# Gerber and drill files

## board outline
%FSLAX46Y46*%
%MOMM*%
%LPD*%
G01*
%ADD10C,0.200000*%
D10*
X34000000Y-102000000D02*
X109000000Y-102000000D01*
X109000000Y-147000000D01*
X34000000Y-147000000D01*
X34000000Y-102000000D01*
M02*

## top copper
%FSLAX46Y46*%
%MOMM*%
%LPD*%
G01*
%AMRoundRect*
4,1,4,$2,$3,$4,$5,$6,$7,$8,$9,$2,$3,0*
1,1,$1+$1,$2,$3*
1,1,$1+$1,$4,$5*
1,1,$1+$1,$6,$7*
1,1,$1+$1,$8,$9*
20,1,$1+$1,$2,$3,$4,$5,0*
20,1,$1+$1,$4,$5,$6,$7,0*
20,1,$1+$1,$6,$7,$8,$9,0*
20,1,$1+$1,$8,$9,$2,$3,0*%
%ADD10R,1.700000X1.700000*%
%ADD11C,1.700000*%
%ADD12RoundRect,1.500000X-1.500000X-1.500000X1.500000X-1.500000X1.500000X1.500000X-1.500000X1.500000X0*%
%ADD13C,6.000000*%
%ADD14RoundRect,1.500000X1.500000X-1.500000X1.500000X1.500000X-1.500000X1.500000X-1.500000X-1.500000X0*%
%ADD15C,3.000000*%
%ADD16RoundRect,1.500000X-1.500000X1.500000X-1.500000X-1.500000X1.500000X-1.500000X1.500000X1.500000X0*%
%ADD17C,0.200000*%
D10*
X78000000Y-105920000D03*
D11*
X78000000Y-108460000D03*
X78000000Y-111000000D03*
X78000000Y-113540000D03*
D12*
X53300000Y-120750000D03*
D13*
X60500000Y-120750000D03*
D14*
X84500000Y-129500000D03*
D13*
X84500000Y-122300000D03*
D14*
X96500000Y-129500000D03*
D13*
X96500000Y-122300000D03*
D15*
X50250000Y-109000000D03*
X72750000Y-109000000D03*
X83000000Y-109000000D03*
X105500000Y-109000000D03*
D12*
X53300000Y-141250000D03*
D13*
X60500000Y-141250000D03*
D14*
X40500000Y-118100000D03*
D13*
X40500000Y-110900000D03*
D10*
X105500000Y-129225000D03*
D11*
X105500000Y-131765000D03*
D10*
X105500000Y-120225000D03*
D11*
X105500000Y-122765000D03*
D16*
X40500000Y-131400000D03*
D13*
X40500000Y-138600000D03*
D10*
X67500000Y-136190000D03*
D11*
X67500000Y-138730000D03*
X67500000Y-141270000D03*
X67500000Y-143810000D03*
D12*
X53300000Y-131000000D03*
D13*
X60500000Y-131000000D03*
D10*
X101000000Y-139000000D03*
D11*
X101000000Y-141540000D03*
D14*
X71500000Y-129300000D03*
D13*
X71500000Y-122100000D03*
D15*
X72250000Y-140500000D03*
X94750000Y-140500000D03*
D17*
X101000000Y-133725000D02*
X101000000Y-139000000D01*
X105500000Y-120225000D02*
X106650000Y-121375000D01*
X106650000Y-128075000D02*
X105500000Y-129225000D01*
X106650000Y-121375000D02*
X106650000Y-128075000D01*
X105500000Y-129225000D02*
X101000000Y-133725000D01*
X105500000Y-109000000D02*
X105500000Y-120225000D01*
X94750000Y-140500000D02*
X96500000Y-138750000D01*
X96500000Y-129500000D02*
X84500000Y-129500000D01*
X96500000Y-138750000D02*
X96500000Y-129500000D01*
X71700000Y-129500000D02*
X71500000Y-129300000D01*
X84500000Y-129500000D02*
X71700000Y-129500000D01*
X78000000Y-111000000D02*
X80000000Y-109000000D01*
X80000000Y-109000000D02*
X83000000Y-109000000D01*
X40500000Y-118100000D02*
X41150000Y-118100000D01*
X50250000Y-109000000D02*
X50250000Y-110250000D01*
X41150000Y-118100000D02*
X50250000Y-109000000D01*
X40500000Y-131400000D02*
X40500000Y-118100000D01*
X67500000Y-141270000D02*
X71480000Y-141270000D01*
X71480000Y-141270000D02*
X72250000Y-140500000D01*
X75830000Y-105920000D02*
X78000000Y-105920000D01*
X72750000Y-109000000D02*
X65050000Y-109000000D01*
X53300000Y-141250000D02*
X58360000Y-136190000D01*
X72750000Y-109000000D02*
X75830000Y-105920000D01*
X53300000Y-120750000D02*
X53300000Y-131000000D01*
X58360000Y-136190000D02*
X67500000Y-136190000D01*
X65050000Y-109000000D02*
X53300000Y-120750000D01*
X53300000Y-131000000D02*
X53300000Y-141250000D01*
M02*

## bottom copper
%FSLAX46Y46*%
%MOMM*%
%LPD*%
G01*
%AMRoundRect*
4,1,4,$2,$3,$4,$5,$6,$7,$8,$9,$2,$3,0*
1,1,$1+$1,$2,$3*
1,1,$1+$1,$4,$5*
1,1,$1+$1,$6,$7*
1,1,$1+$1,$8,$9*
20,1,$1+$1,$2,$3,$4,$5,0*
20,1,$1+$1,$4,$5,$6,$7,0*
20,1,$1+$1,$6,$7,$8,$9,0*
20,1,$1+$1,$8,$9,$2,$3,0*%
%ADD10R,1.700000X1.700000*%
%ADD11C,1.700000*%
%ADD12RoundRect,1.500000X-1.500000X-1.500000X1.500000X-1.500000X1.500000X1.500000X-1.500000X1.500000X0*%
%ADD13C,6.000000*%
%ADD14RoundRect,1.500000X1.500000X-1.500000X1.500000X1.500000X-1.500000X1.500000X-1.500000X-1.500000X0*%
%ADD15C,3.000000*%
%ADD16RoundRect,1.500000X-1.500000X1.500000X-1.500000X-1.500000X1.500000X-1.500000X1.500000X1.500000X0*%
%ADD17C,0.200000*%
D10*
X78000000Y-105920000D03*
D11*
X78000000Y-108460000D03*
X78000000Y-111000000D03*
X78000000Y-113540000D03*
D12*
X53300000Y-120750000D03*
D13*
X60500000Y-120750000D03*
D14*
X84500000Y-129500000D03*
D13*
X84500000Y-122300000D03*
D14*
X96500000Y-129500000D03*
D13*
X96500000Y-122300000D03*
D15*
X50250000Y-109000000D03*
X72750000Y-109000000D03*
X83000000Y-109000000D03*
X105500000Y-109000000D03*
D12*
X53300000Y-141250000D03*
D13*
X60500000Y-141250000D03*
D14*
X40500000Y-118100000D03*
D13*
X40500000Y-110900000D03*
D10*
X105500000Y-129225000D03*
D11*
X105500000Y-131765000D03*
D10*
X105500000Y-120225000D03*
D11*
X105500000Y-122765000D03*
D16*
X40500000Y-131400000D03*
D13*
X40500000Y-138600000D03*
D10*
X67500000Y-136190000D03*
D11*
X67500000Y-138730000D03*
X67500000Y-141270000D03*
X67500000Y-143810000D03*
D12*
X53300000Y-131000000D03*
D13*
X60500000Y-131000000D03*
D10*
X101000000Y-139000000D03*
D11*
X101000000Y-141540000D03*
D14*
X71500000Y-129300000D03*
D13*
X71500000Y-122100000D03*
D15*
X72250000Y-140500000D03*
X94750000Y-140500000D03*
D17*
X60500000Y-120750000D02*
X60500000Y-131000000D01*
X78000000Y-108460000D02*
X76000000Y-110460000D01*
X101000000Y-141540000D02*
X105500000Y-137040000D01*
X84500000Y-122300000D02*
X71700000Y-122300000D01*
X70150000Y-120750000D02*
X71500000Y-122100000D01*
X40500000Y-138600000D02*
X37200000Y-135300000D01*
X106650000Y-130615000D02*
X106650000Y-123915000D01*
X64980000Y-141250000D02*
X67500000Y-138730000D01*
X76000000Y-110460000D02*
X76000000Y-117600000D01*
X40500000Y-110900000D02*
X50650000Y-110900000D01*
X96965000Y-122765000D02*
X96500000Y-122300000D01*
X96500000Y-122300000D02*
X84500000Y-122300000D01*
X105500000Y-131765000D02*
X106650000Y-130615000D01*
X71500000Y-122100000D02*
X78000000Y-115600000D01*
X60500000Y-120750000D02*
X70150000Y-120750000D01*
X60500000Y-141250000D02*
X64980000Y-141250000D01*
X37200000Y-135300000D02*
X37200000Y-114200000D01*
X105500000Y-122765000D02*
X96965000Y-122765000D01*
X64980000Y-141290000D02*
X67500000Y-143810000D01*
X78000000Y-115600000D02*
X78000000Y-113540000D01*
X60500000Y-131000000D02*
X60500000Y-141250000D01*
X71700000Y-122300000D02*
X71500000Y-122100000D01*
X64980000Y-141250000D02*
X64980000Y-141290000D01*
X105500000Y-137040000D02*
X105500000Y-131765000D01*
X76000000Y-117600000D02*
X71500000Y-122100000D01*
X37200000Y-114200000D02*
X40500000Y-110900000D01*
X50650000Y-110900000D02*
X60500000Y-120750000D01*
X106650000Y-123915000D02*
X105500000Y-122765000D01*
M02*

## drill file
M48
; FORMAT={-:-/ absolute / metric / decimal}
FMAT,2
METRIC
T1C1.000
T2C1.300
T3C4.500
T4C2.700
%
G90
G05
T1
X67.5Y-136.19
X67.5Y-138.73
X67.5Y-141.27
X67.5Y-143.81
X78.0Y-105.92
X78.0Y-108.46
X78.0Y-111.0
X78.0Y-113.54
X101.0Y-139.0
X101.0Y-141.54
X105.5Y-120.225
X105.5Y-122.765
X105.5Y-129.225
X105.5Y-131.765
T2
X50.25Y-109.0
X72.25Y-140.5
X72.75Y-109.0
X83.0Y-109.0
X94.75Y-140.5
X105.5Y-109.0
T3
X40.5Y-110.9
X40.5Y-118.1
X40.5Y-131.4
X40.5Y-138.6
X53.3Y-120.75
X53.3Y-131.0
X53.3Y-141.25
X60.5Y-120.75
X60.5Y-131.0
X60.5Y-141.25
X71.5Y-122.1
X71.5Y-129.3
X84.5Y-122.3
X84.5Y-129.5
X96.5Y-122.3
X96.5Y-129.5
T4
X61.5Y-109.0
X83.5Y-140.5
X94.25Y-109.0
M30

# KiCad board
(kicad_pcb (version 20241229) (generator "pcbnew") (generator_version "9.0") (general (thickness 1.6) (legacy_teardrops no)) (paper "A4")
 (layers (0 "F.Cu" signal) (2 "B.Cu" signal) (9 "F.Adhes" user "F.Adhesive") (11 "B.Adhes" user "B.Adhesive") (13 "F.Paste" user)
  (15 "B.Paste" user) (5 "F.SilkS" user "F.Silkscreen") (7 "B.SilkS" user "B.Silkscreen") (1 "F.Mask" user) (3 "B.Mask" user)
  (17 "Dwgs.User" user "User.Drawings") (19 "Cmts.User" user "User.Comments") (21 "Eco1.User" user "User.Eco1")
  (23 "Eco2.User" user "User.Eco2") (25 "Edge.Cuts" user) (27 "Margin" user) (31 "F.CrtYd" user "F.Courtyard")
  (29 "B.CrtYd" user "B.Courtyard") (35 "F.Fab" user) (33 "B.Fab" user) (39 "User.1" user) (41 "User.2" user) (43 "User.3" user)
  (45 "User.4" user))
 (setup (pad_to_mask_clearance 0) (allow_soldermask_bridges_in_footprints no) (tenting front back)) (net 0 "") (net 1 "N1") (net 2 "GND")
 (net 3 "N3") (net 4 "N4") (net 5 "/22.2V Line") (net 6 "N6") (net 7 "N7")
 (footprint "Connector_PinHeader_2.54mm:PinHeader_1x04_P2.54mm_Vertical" (layer "F.Cu") (at 78 105.92)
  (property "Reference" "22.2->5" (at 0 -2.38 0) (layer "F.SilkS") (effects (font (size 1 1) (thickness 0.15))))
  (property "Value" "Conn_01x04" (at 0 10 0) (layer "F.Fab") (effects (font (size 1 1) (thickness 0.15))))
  (pad "1" thru_hole rect (at 0 0) (size 1.7 1.7) (drill 1) (layers "*.Cu" "*.Mask") (remove_unused_layers no) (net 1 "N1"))
  (pad "2" thru_hole circle (at 0 2.54) (size 1.7 1.7) (drill 1) (layers "*.Cu" "*.Mask") (remove_unused_layers no) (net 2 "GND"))
  (pad "3" thru_hole circle (at 0 5.08) (size 1.7 1.7) (drill 1) (layers "*.Cu" "*.Mask") (remove_unused_layers no) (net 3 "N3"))
  (pad "4" thru_hole circle (at 0 7.62) (size 1.7 1.7) (drill 1) (layers "*.Cu" "*.Mask") (remove_unused_layers no) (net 2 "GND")))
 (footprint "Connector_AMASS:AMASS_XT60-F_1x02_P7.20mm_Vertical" (layer "F.Cu") (at 53.3 120.75)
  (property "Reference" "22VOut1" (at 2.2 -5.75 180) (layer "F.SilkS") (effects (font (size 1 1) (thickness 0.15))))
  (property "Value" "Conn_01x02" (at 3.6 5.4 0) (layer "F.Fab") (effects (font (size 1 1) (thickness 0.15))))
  (pad "1" thru_hole roundrect (at 0 0) (size 6 6) (drill 4.5) (layers "*.Cu" "*.Mask") (remove_unused_layers no) (roundrect_rratio 0.25)
   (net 1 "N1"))
  (pad "2" thru_hole circle (at 7.2 0) (size 6 6) (drill 4.5) (layers "*.Cu" "*.Mask") (remove_unused_layers no) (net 2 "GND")))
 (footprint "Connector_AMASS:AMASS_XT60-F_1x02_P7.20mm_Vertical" (layer "F.Cu") (at 84.5 129.5 90)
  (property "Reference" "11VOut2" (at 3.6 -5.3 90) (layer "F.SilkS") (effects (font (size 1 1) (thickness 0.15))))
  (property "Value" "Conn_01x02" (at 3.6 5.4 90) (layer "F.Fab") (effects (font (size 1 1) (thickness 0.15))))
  (pad "1" thru_hole roundrect (at 0 0 90) (size 6 6) (drill 4.5) (layers "*.Cu" "*.Mask") (remove_unused_layers no) (roundrect_rratio 0.25)
   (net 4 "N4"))
  (pad "2" thru_hole circle (at 7.2 0 90) (size 6 6) (drill 4.5) (layers "*.Cu" "*.Mask") (remove_unused_layers no) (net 2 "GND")))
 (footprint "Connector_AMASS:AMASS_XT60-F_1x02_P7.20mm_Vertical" (layer "F.Cu") (at 96.5 129.5 90)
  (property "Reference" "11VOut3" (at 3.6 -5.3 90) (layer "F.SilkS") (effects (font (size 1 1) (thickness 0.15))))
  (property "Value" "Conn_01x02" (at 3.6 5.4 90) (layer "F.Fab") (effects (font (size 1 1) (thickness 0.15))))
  (pad "1" thru_hole roundrect (at 0 0 90) (size 6 6) (drill 4.5) (layers "*.Cu" "*.Mask") (remove_unused_layers no) (roundrect_rratio 0.25)
   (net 4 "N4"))
  (pad "2" thru_hole circle (at 7.2 0 90) (size 6 6) (drill 4.5) (layers "*.Cu" "*.Mask") (remove_unused_layers no) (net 2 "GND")))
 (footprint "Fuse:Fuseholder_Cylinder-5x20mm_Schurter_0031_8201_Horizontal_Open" (layer "F.Cu") (at 50.25 109)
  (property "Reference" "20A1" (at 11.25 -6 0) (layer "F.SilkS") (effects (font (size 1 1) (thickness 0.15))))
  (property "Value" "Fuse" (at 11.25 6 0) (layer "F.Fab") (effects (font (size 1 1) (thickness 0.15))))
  (pad "" np_thru_hole circle (at 11.25 0) (size 2.7 2.7) (drill 2.7) (layers "*.Cu" "*.Mask"))
  (pad "1" thru_hole circle (at 0 0) (size 3 3) (drill 1.3) (layers "*.Cu" "*.Mask") (remove_unused_layers no) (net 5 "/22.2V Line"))
  (pad "2" thru_hole circle (at 22.5 0) (size 3 3) (drill 1.3) (layers "*.Cu" "*.Mask") (remove_unused_layers no) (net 1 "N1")))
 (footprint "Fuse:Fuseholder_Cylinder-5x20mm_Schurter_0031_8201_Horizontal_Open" (layer "F.Cu") (at 83 109)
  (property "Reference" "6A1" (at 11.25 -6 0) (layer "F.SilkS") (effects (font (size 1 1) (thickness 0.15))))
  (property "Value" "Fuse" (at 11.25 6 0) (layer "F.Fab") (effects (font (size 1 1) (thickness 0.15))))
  (pad "" np_thru_hole circle (at 11.25 0) (size 2.7 2.7) (drill 2.7) (layers "*.Cu" "*.Mask"))
  (pad "1" thru_hole circle (at 0 0) (size 3 3) (drill 1.3) (layers "*.Cu" "*.Mask") (remove_unused_layers no) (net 3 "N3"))
  (pad "2" thru_hole circle (at 22.5 0) (size 3 3) (drill 1.3) (layers "*.Cu" "*.Mask") (remove_unused_layers no) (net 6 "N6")))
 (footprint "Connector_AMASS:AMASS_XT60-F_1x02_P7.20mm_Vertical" (layer "F.Cu") (at 53.3 141.25)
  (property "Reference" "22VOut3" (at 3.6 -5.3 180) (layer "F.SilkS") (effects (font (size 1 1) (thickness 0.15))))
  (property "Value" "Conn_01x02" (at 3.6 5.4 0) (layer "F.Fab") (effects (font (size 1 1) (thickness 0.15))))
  (pad "1" thru_hole roundrect (at 0 0) (size 6 6) (drill 4.5) (layers "*.Cu" "*.Mask") (remove_unused_layers no) (roundrect_rratio 0.25)
   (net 1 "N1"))
  (pad "2" thru_hole circle (at 7.2 0) (size 6 6) (drill 4.5) (layers "*.Cu" "*.Mask") (remove_unused_layers no) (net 2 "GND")))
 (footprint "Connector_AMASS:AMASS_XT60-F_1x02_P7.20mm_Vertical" (layer "F.Cu") (at 40.5 118.1 90)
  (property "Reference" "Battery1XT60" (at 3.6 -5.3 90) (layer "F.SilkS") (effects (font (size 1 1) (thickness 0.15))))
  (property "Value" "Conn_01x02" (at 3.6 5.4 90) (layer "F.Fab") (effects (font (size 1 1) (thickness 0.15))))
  (pad "1" thru_hole roundrect (at 0 0 90) (size 6 6) (drill 4.5) (layers "*.Cu" "*.Mask") (remove_unused_layers no) (roundrect_rratio 0.25)
   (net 5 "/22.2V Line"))
  (pad "2" thru_hole circle (at 7.2 0 90) (size 6 6) (drill 4.5) (layers "*.Cu" "*.Mask") (remove_unused_layers no) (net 2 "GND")))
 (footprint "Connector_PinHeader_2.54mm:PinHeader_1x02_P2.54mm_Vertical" (layer "F.Cu") (at 105.5 129.225)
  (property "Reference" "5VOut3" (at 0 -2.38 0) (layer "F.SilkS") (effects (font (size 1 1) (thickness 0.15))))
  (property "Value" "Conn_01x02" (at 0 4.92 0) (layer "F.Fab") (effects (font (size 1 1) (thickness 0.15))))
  (pad "1" thru_hole rect (at 0 0) (size 1.7 1.7) (drill 1) (layers "*.Cu" "*.Mask") (remove_unused_layers no) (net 6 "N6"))
  (pad "2" thru_hole circle (at 0 2.54) (size 1.7 1.7) (drill 1) (layers "*.Cu" "*.Mask") (remove_unused_layers no) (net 2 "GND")))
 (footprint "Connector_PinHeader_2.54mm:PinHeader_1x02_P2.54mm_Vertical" (layer "F.Cu") (at 105.5 120.225)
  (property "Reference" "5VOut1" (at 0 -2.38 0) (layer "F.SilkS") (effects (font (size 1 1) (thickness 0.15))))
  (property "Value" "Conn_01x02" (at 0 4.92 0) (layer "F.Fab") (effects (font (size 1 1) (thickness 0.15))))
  (pad "1" thru_hole rect (at 0 0) (size 1.7 1.7) (drill 1) (layers "*.Cu" "*.Mask") (remove_unused_layers no) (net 6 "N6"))
  (pad "2" thru_hole circle (at 0 2.54) (size 1.7 1.7) (drill 1) (layers "*.Cu" "*.Mask") (remove_unused_layers no) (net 2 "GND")))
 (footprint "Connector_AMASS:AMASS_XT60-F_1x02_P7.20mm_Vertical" (layer "F.Cu") (at 40.5 131.4 -90)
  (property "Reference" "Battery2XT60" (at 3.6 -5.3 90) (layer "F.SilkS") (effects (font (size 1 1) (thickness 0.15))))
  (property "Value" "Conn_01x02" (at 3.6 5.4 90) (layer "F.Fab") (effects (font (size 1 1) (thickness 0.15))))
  (pad "1" thru_hole roundrect (at 0 0 270) (size 6 6) (drill 4.5) (layers "*.Cu" "*.Mask") (remove_unused_layers no)
   (roundrect_rratio 0.25) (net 5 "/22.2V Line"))
  (pad "2" thru_hole circle (at 7.2 0 270) (size 6 6) (drill 4.5) (layers "*.Cu" "*.Mask") (remove_unused_layers no) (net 2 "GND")))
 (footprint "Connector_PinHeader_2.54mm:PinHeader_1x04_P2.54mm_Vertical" (layer "F.Cu") (at 67.5 136.19)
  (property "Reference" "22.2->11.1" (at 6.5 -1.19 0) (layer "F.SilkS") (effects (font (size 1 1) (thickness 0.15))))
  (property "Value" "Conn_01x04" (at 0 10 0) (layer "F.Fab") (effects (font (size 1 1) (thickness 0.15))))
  (pad "1" thru_hole rect (at 0 0) (size 1.7 1.7) (drill 1) (layers "*.Cu" "*.Mask") (remove_unused_layers no) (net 1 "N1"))
  (pad "2" thru_hole circle (at 0 2.54) (size 1.7 1.7) (drill 1) (layers "*.Cu" "*.Mask") (remove_unused_layers no) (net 2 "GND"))
  (pad "3" thru_hole circle (at 0 5.08) (size 1.7 1.7) (drill 1) (layers "*.Cu" "*.Mask") (remove_unused_layers no) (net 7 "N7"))
  (pad "4" thru_hole circle (at 0 7.62) (size 1.7 1.7) (drill 1) (layers "*.Cu" "*.Mask") (remove_unused_layers no) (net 2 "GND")))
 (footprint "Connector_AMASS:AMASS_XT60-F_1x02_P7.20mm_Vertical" (layer "F.Cu") (at 53.3 131)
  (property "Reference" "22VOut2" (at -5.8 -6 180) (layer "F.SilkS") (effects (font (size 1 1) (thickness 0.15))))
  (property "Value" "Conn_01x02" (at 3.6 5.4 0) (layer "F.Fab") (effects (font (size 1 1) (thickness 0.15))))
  (pad "1" thru_hole roundrect (at 0 0) (size 6 6) (drill 4.5) (layers "*.Cu" "*.Mask") (remove_unused_layers no) (roundrect_rratio 0.25)
   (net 1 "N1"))
  (pad "2" thru_hole circle (at 7.2 0) (size 6 6) (drill 4.5) (layers "*.Cu" "*.Mask") (remove_unused_layers no) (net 2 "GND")))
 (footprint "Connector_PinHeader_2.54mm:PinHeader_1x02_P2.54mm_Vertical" (layer "F.Cu") (at 101 139)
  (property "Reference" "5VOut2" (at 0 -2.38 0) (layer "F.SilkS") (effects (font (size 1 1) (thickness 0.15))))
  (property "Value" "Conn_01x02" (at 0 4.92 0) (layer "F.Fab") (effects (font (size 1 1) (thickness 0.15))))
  (pad "1" thru_hole rect (at 0 0) (size 1.7 1.7) (drill 1) (layers "*.Cu" "*.Mask") (remove_unused_layers no) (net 6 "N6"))
  (pad "2" thru_hole circle (at 0 2.54) (size 1.7 1.7) (drill 1) (layers "*.Cu" "*.Mask") (remove_unused_layers no) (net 2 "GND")))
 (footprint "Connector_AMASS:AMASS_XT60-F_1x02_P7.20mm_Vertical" (layer "F.Cu") (at 71.5 129.3 90)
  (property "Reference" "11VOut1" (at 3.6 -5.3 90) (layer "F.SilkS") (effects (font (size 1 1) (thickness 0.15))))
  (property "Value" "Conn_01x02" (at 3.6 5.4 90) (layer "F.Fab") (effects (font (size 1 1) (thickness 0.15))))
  (pad "1" thru_hole roundrect (at 0 0 90) (size 6 6) (drill 4.5) (layers "*.Cu" "*.Mask") (remove_unused_layers no) (roundrect_rratio 0.25)
   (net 4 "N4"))
  (pad "2" thru_hole circle (at 7.2 0 90) (size 6 6) (drill 4.5) (layers "*.Cu" "*.Mask") (remove_unused_layers no) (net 2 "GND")))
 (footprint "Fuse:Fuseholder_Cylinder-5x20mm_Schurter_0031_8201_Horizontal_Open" (layer "F.Cu") (at 72.25 140.5)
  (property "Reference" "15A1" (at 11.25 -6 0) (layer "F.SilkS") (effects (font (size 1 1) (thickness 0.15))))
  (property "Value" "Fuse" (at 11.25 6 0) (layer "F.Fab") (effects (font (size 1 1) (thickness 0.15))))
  (pad "" np_thru_hole circle (at 11.25 0) (size 2.7 2.7) (drill 2.7) (layers "*.Cu" "*.Mask"))
  (pad "1" thru_hole circle (at 0 0) (size 3 3) (drill 1.3) (layers "*.Cu" "*.Mask") (remove_unused_layers no) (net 7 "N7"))
  (pad "2" thru_hole circle (at 22.5 0) (size 3 3) (drill 1.3) (layers "*.Cu" "*.Mask") (remove_unused_layers no) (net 4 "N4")))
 (gr_rect (start 34 102) (end 109 147) (stroke (width 0.2) (type solid)) (fill no) (layer "Edge.Cuts"))
 (segment (start 60.5 120.75) (end 60.5 131) (width 0.2) (layer "B.Cu") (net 2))
 (segment (start 78 108.46) (end 76 110.46) (width 0.2) (layer "B.Cu") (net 2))
 (segment (start 101 141.54) (end 105.5 137.04) (width 0.2) (layer "B.Cu") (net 2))
 (segment (start 84.5 122.3) (end 71.7 122.3) (width 0.2) (layer "B.Cu") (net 2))
 (segment (start 70.15 120.75) (end 71.5 122.1) (width 0.2) (layer "B.Cu") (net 2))
 (segment (start 40.5 138.6) (end 37.2 135.3) (width 0.2) (layer "B.Cu") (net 2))
 (segment (start 106.65 130.615) (end 106.65 123.915) (width 0.2) (layer "B.Cu") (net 2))
 (segment (start 64.98 141.25) (end 67.5 138.73) (width 0.2) (layer "B.Cu") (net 2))
 (segment (start 76 110.46) (end 76 117.6) (width 0.2) (layer "B.Cu") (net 2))
 (segment (start 40.5 110.9) (end 50.65 110.9) (width 0.2) (layer "B.Cu") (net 2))
 (segment (start 96.965 122.765) (end 96.5 122.3) (width 0.2) (layer "B.Cu") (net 2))
 (segment (start 96.5 122.3) (end 84.5 122.3) (width 0.2) (layer "B.Cu") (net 2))
 (segment (start 105.5 131.765) (end 106.65 130.615) (width 0.2) (layer "B.Cu") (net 2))
 (segment (start 71.5 122.1) (end 78 115.6) (width 0.2) (layer "B.Cu") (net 2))
 (segment (start 60.5 120.75) (end 70.15 120.75) (width 0.2) (layer "B.Cu") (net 2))
 (segment (start 60.5 141.25) (end 64.98 141.25) (width 0.2) (layer "B.Cu") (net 2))
 (segment (start 37.2 135.3) (end 37.2 114.2) (width 0.2) (layer "B.Cu") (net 2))
 (segment (start 105.5 122.765) (end 96.965 122.765) (width 0.2) (layer "B.Cu") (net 2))
 (segment (start 64.98 141.29) (end 67.5 143.81) (width 0.2) (layer "B.Cu") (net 2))
 (segment (start 78 115.6) (end 78 113.54) (width 0.2) (layer "B.Cu") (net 2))
 (segment (start 60.5 131) (end 60.5 141.25) (width 0.2) (layer "B.Cu") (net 2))
 (segment (start 71.7 122.3) (end 71.5 122.1) (width 0.2) (layer "B.Cu") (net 2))
 (segment (start 64.98 141.25) (end 64.98 141.29) (width 0.2) (layer "B.Cu") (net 2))
 (segment (start 105.5 137.04) (end 105.5 131.765) (width 0.2) (layer "B.Cu") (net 2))
 (segment (start 76 117.6) (end 71.5 122.1) (width 0.2) (layer "B.Cu") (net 2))
 (segment (start 37.2 114.2) (end 40.5 110.9) (width 0.2) (layer "B.Cu") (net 2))
 (segment (start 50.65 110.9) (end 60.5 120.75) (width 0.2) (layer "B.Cu") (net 2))
 (segment (start 106.65 123.915) (end 105.5 122.765) (width 0.2) (layer "B.Cu") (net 2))
 (segment (start 101 133.725) (end 101 139) (width 0.2) (layer "F.Cu") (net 6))
 (segment (start 105.5 120.225) (end 106.65 121.375) (width 0.2) (layer "F.Cu") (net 6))
 (segment (start 106.65 128.075) (end 105.5 129.225) (width 0.2) (layer "F.Cu") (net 6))
 (segment (start 106.65 121.375) (end 106.65 128.075) (width 0.2) (layer "F.Cu") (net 6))
 (segment (start 105.5 129.225) (end 101 133.725) (width 0.2) (layer "F.Cu") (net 6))
 (segment (start 105.5 109) (end 105.5 120.225) (width 0.2) (layer "F.Cu") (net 6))
 (segment (start 94.75 140.5) (end 96.5 138.75) (width 0.2) (layer "F.Cu") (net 4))
 (segment (start 96.5 129.5) (end 84.5 129.5) (width 0.2) (layer "F.Cu") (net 4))
 (segment (start 96.5 138.75) (end 96.5 129.5) (width 0.2) (layer "F.Cu") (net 4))
 (segment (start 71.7 129.5) (end 71.5 129.3) (width 0.2) (layer "F.Cu") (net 4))
 (segment (start 84.5 129.5) (end 71.7 129.5) (width 0.2) (layer "F.Cu") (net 4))
 (segment (start 78 111) (end 80 109) (width 0.2) (layer "F.Cu") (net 3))
 (segment (start 80 109) (end 83 109) (width 0.2) (layer "F.Cu") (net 3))
 (segment (start 40.5 118.1) (end 41.15 118.1) (width 0.2) (layer "F.Cu") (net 5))
 (segment (start 50.25 109) (end 50.25 110.25) (width 0.2) (layer "F.Cu") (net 5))
 (segment (start 41.15 118.1) (end 50.25 109) (width 0.2) (layer "F.Cu") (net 5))
 (segment (start 40.5 131.4) (end 40.5 118.1) (width 0.2) (layer "F.Cu") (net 5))
 (segment (start 67.5 141.27) (end 71.48 141.27) (width 0.2) (layer "F.Cu") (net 7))
 (segment (start 71.48 141.27) (end 72.25 140.5) (width 0.2) (layer "F.Cu") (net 7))
 (segment (start 75.83 105.92) (end 78 105.92) (width 0.2) (layer "F.Cu") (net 1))
 (segment (start 72.75 109) (end 65.05 109) (width 0.2) (layer "F.Cu") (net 1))
 (segment (start 53.3 141.25) (end 58.36 136.19) (width 0.2) (layer "F.Cu") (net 1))
 (segment (start 72.75 109) (end 75.83 105.92) (width 0.2) (layer "F.Cu") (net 1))
 (segment (start 53.3 120.75) (end 53.3 131) (width 0.2) (layer "F.Cu") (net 1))
 (segment (start 58.36 136.19) (end 67.5 136.19) (width 0.2) (layer "F.Cu") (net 1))
 (segment (start 65.05 109) (end 53.3 120.75) (width 0.2) (layer "F.Cu") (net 1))
 (segment (start 53.3 131) (end 53.3 141.25) (width 0.2) (layer "F.Cu") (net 1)))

